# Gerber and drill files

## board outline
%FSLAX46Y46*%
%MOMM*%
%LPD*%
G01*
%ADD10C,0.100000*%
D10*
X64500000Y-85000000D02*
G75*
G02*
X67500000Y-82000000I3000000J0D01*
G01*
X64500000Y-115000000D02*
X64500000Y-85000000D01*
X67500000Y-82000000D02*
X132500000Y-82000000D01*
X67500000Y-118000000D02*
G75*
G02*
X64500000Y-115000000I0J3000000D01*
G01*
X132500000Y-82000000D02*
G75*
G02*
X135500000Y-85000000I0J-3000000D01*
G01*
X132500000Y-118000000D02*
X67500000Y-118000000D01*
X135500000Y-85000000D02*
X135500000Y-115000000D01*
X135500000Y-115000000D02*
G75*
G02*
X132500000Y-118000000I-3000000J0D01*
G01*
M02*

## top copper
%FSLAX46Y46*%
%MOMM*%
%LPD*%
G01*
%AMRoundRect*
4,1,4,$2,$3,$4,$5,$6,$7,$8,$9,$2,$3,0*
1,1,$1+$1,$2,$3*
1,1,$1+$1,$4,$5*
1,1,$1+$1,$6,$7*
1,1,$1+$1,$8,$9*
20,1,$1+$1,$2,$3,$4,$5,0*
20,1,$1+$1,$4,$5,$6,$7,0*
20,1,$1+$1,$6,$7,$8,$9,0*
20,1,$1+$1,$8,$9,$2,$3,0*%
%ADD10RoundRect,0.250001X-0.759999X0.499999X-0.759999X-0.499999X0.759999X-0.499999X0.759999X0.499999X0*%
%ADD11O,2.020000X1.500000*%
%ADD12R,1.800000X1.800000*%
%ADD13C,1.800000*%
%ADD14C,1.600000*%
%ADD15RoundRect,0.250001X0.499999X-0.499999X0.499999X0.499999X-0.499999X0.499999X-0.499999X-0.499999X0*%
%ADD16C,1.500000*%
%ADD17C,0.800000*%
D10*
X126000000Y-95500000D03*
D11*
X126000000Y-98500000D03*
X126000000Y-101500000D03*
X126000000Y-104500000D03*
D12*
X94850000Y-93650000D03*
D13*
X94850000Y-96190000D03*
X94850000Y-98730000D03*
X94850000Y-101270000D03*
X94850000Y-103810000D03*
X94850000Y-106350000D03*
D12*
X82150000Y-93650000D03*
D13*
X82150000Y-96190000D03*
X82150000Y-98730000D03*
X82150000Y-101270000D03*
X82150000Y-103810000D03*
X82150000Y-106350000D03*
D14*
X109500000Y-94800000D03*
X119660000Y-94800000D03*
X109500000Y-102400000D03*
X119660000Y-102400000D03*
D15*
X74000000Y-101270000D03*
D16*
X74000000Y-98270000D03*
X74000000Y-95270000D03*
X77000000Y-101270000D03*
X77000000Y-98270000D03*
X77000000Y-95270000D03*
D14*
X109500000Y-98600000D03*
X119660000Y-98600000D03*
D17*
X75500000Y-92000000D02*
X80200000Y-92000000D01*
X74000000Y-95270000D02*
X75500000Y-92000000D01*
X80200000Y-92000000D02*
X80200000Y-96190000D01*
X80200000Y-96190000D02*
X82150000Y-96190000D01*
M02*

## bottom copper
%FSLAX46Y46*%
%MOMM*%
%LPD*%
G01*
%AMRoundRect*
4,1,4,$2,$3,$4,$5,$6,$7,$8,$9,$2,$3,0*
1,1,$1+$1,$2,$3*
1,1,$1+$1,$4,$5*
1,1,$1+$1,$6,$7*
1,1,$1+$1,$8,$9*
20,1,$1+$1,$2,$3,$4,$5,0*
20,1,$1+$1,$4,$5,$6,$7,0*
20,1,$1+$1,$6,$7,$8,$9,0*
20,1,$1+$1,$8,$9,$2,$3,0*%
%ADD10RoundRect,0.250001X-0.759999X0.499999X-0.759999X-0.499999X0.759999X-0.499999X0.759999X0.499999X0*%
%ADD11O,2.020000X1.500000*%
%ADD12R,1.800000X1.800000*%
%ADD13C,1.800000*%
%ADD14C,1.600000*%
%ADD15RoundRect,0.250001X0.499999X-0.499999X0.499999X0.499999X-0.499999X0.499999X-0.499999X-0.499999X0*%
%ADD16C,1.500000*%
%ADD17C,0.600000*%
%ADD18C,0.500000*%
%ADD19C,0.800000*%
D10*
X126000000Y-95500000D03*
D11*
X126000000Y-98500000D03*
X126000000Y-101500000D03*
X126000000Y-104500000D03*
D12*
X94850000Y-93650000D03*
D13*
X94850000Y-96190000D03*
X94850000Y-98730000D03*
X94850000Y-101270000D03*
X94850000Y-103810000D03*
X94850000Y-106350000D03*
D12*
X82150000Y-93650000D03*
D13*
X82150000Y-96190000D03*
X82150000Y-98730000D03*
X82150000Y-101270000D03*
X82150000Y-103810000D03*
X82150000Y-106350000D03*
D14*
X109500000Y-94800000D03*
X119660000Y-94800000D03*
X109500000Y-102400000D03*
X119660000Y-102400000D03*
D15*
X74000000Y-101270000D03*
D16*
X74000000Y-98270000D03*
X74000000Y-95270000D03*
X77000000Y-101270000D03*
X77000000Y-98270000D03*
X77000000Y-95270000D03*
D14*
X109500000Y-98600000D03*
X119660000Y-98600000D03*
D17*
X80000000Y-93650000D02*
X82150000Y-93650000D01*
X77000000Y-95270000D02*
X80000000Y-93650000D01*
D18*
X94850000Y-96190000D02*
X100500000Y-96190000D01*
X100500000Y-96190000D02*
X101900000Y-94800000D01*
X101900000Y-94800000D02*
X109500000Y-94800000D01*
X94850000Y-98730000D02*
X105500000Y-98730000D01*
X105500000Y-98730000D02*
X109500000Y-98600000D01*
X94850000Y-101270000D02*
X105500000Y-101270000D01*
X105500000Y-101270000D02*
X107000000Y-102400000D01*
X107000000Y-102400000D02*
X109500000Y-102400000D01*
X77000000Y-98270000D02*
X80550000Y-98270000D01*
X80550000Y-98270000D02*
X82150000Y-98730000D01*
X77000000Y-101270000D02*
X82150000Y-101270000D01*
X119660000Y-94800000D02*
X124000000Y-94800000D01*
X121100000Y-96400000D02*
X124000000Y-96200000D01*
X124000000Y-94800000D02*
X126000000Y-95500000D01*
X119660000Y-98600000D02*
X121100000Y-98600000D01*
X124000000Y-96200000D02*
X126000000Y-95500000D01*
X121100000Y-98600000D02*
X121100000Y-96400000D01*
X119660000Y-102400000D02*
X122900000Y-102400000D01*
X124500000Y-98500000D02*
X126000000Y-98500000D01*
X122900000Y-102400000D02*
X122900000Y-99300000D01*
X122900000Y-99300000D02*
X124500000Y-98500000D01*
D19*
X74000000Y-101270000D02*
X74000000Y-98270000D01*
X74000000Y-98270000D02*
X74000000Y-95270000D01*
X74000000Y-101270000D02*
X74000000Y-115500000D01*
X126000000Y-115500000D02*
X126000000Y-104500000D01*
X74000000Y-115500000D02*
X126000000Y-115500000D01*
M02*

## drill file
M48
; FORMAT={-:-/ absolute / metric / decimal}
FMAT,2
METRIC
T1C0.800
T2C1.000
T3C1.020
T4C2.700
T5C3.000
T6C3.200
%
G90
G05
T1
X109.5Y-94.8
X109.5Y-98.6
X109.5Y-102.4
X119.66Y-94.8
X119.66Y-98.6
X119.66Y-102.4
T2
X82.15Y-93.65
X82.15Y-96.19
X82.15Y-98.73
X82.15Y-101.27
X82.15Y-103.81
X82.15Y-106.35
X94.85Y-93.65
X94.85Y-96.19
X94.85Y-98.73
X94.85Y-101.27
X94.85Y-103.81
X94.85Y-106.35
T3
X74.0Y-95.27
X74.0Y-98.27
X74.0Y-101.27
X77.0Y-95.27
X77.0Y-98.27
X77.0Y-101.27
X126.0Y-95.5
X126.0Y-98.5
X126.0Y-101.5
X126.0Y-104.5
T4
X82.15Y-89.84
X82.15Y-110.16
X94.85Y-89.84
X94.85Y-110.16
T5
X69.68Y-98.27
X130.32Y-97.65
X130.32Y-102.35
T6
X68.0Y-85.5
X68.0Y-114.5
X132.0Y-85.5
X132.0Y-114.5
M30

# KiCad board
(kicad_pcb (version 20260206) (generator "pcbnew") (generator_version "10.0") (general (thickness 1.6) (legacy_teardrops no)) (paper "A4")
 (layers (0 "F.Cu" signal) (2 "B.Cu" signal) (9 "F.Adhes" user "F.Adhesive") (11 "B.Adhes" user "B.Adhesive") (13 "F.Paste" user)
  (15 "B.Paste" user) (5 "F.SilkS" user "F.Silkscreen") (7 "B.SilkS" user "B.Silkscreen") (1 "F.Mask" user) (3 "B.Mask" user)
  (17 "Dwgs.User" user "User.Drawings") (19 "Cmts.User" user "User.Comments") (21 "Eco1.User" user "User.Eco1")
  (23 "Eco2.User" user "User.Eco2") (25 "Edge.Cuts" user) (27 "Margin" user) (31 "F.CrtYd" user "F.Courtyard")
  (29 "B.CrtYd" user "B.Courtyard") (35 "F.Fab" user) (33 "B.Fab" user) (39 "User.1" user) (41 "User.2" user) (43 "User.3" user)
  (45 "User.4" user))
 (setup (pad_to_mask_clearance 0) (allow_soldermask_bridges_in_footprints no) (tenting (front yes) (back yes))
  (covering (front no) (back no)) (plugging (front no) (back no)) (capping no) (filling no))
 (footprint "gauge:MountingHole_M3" (layer "F.Cu") (at 68 114.5)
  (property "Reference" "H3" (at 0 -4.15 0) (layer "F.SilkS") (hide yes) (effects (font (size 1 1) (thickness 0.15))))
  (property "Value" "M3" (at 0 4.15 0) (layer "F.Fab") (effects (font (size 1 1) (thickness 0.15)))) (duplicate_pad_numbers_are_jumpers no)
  (pad "" np_thru_hole circle (at 0 0) (size 3.2 3.2) (drill 3.2) (layers "*.Cu" "*.Mask")))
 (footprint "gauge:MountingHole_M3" (layer "F.Cu") (at 68 85.5)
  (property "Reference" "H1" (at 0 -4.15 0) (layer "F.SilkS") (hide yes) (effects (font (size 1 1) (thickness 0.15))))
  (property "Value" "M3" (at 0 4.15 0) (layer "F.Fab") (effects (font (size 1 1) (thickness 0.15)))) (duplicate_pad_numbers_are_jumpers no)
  (pad "" np_thru_hole circle (at 0 0) (size 3.2 3.2) (drill 3.2) (layers "*.Cu" "*.Mask")))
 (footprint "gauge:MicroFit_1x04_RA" (layer "F.Cu") (at 126 95.5 -90)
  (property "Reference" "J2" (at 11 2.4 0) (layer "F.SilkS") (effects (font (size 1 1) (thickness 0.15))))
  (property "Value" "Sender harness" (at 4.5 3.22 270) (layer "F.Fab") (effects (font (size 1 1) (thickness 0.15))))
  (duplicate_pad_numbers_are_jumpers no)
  (pad "" np_thru_hole circle (at 2.15 -4.32 270) (size 3 3) (drill 3) (layers "*.Cu" "*.Mask"))
  (pad "" np_thru_hole circle (at 6.85 -4.32 270) (size 3 3) (drill 3) (layers "*.Cu" "*.Mask"))
  (pad "1" thru_hole roundrect (at 0 0 270) (size 1.5 2.02) (drill 1.02) (layers "*.Cu" "*.Mask") (remove_unused_layers no)
   (roundrect_rratio 0.166667) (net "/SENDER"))
  (pad "2" thru_hole oval (at 3 0 270) (size 1.5 2.02) (drill 1.02) (layers "*.Cu" "*.Mask") (remove_unused_layers no) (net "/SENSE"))
  (pad "3" thru_hole oval (at 6 0 270) (size 1.5 2.02) (drill 1.02) (layers "*.Cu" "*.Mask") (remove_unused_layers no)
   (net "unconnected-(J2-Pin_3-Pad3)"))
  (pad "4" thru_hole oval (at 9 0 270) (size 1.5 2.02) (drill 1.02) (layers "*.Cu" "*.Mask") (remove_unused_layers no) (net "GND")))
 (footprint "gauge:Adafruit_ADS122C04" (layer "F.Cu") (at 88.5 100 -90)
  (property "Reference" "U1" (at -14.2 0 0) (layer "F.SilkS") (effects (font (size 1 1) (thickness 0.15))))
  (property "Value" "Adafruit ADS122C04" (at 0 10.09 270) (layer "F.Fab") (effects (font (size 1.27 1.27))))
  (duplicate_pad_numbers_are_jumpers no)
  (pad "" np_thru_hole circle (at -10.16 -6.35 270) (size 2.7 2.7) (drill 2.7) (layers "*.Cu"))
  (pad "" np_thru_hole circle (at -10.16 6.35 270) (size 2.7 2.7) (drill 2.7) (layers "*.Cu"))
  (pad "" np_thru_hole circle (at 10.16 -6.35 270) (size 2.7 2.7) (drill 2.7) (layers "*.Cu"))
  (pad "" np_thru_hole circle (at 10.16 6.35 270) (size 2.7 2.7) (drill 2.7) (layers "*.Cu"))
  (pad "1" thru_hole rect (at -6.35 -6.35 270) (size 1.8 1.8) (drill 1) (layers "*.Cu" "*.Mask") (remove_unused_layers no)
   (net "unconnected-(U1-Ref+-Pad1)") (thermal_bridge_angle 45))
  (pad "2" thru_hole circle (at -3.81 -6.35 270) (size 1.8 1.8) (drill 1) (layers "*.Cu" "*.Mask") (remove_unused_layers no) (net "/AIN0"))
  (pad "3" thru_hole circle (at -1.27 -6.35 270) (size 1.8 1.8) (drill 1) (layers "*.Cu" "*.Mask") (remove_unused_layers no) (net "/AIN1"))
  (pad "4" thru_hole circle (at 1.27 -6.35 270) (size 1.8 1.8) (drill 1) (layers "*.Cu" "*.Mask") (remove_unused_layers no) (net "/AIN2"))
  (pad "5" thru_hole circle (at 3.81 -6.35 270) (size 1.8 1.8) (drill 1) (layers "*.Cu" "*.Mask") (remove_unused_layers no)
   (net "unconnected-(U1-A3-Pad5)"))
  (pad "6" thru_hole circle (at 6.35 -6.35 270) (size 1.8 1.8) (drill 1) (layers "*.Cu" "*.Mask") (remove_unused_layers no)
   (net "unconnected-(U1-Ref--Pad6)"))
  (pad "7" thru_hole rect (at -6.35 6.35 270) (size 1.8 1.8) (drill 1) (layers "*.Cu" "*.Mask") (remove_unused_layers no) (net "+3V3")
   (thermal_bridge_angle 45))
  (pad "8" thru_hole circle (at -3.81 6.35 270) (size 1.8 1.8) (drill 1) (layers "*.Cu" "*.Mask") (remove_unused_layers no) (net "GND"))
  (pad "9" thru_hole circle (at -1.27 6.35 270) (size 1.8 1.8) (drill 1) (layers "*.Cu" "*.Mask") (remove_unused_layers no) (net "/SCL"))
  (pad "10" thru_hole circle (at 1.27 6.35 270) (size 1.8 1.8) (drill 1) (layers "*.Cu" "*.Mask") (remove_unused_layers no) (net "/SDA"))
  (pad "11" thru_hole circle (at 3.81 6.35 270) (size 1.8 1.8) (drill 1) (layers "*.Cu" "*.Mask") (remove_unused_layers no)
   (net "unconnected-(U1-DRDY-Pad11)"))
  (pad "12" thru_hole circle (at 6.35 6.35 270) (size 1.8 1.8) (drill 1) (layers "*.Cu" "*.Mask") (remove_unused_layers no)
   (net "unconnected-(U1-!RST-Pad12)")))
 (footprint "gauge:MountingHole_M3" (layer "F.Cu") (at 132 114.5)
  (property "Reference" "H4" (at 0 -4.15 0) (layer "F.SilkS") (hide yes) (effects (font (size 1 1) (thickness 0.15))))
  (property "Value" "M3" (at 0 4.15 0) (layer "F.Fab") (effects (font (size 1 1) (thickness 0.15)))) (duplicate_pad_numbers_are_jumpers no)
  (pad "" np_thru_hole circle (at 0 0) (size 3.2 3.2) (drill 3.2) (layers "*.Cu" "*.Mask")))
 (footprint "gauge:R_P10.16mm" (layer "F.Cu") (at 109.5 94.8)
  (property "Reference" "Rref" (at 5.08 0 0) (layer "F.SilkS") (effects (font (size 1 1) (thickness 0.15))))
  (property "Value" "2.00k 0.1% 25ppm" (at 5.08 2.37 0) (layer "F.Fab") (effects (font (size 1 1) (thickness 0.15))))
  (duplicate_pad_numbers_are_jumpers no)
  (pad "1" thru_hole circle (at 0 0) (size 1.6 1.6) (drill 0.8) (layers "*.Cu" "*.Mask") (remove_unused_layers no) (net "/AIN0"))
  (pad "2" thru_hole circle (at 10.16 0) (size 1.6 1.6) (drill 0.8) (layers "*.Cu" "*.Mask") (remove_unused_layers no) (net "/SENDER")))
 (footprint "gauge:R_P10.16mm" (layer "F.Cu") (at 109.5 102.4)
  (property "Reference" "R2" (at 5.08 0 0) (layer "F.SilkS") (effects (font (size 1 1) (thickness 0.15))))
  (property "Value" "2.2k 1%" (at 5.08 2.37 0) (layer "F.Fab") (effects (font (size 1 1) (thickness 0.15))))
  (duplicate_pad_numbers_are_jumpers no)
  (pad "1" thru_hole circle (at 0 0) (size 1.6 1.6) (drill 0.8) (layers "*.Cu" "*.Mask") (remove_unused_layers no) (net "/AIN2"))
  (pad "2" thru_hole circle (at 10.16 0) (size 1.6 1.6) (drill 0.8) (layers "*.Cu" "*.Mask") (remove_unused_layers no) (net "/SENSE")))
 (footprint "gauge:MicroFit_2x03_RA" (layer "F.Cu") (at 74 101.27 90)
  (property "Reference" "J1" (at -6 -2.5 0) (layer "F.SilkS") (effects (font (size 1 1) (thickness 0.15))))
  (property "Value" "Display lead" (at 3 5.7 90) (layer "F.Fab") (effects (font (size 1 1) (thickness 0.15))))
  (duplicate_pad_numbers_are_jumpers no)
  (pad "" np_thru_hole circle (at 3 -4.32 90) (size 3 3) (drill 3) (layers "*.Cu" "*.Mask"))
  (pad "1" thru_hole roundrect (at 0 0 90) (size 1.5 1.5) (drill 1.02) (layers "*.Cu" "*.Mask") (remove_unused_layers no)
   (roundrect_rratio 0.166667) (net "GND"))
  (pad "2" thru_hole circle (at 3 0 90) (size 1.5 1.5) (drill 1.02) (layers "*.Cu" "*.Mask") (remove_unused_layers no) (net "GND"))
  (pad "3" thru_hole circle (at 6 0 90) (size 1.5 1.5) (drill 1.02) (layers "*.Cu" "*.Mask") (remove_unused_layers no) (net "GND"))
  (pad "4" thru_hole circle (at 0 3 90) (size 1.5 1.5) (drill 1.02) (layers "*.Cu" "*.Mask") (remove_unused_layers no) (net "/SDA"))
  (pad "5" thru_hole circle (at 3 3 90) (size 1.5 1.5) (drill 1.02) (layers "*.Cu" "*.Mask") (remove_unused_layers no) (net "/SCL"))
  (pad "6" thru_hole circle (at 6 3 90) (size 1.5 1.5) (drill 1.02) (layers "*.Cu" "*.Mask") (remove_unused_layers no) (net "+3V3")))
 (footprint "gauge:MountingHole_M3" (layer "F.Cu") (at 132 85.5)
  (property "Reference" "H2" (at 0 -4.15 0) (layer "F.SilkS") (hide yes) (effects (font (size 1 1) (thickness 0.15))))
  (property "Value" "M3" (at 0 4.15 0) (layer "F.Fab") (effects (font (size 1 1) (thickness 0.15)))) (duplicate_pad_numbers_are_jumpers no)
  (pad "" np_thru_hole circle (at 0 0) (size 3.2 3.2) (drill 3.2) (layers "*.Cu" "*.Mask")))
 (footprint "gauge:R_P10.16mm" (layer "F.Cu") (at 109.5 98.6)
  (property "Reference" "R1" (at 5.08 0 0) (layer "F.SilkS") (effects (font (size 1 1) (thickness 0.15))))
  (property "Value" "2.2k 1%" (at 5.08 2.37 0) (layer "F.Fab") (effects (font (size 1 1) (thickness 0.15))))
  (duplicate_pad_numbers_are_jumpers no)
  (pad "1" thru_hole circle (at 0 0) (size 1.6 1.6) (drill 0.8) (layers "*.Cu" "*.Mask") (remove_unused_layers no) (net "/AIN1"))
  (pad "2" thru_hole circle (at 10.16 0) (size 1.6 1.6) (drill 0.8) (layers "*.Cu" "*.Mask") (remove_unused_layers no) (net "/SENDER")))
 (gr_arc (start 64.5 85) (mid 65.37868 82.87868) (end 67.5 82) (stroke (width 0.1) (type default)) (layer "Edge.Cuts"))
 (gr_line (start 64.5 115) (end 64.5 85) (stroke (width 0.1) (type default)) (layer "Edge.Cuts"))
 (gr_line (start 67.5 82) (end 132.5 82) (stroke (width 0.1) (type default)) (layer "Edge.Cuts"))
 (gr_arc (start 67.5 118) (mid 65.37868 117.12132) (end 64.5 115) (stroke (width 0.1) (type default)) (layer "Edge.Cuts"))
 (gr_arc (start 132.5 82) (mid 134.62132 82.87868) (end 135.5 85) (stroke (width 0.1) (type default)) (layer "Edge.Cuts"))
 (gr_line (start 132.5 118) (end 67.5 118) (stroke (width 0.1) (type default)) (layer "Edge.Cuts"))
 (gr_line (start 135.5 85) (end 135.5 115) (stroke (width 0.1) (type default)) (layer "Edge.Cuts"))
 (gr_arc (start 135.5 115) (mid 134.62132 117.12132) (end 132.5 118) (stroke (width 0.1) (type default)) (layer "Edge.Cuts"))
 (segment (start 80 93.65) (end 82.15 93.65) (width 0.6) (layer "B.Cu") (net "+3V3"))
 (segment (start 77 95.27) (end 80 93.65) (width 0.6) (layer "B.Cu") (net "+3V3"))
 (segment (start 94.85 96.19) (end 100.5 96.19) (width 0.5) (layer "B.Cu") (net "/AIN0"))
 (segment (start 100.5 96.19) (end 101.9 94.8) (width 0.5) (layer "B.Cu") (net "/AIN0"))
 (segment (start 101.9 94.8) (end 109.5 94.8) (width 0.5) (layer "B.Cu") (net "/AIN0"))
 (segment (start 94.85 98.73) (end 105.5 98.73) (width 0.5) (layer "B.Cu") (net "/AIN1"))
 (segment (start 105.5 98.73) (end 109.5 98.6) (width 0.5) (layer "B.Cu") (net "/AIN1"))
 (segment (start 94.85 101.27) (end 105.5 101.27) (width 0.5) (layer "B.Cu") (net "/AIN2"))
 (segment (start 105.5 101.27) (end 107 102.4) (width 0.5) (layer "B.Cu") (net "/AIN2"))
 (segment (start 107 102.4) (end 109.5 102.4) (width 0.5) (layer "B.Cu") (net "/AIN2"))
 (segment (start 77 98.27) (end 80.55 98.27) (width 0.5) (layer "B.Cu") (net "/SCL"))
 (segment (start 80.55 98.27) (end 82.15 98.73) (width 0.5) (layer "B.Cu") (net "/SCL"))
 (segment (start 77 101.27) (end 82.15 101.27) (width 0.5) (layer "B.Cu") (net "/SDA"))
 (segment (start 119.66 94.8) (end 124 94.8) (width 0.5) (layer "B.Cu") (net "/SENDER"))
 (segment (start 121.1 96.4) (end 124 96.2) (width 0.5) (layer "B.Cu") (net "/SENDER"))
 (segment (start 124 94.8) (end 126 95.5) (width 0.5) (layer "B.Cu") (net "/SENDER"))
 (segment (start 119.66 98.6) (end 121.1 98.6) (width 0.5) (layer "B.Cu") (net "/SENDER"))
 (segment (start 124 96.2) (end 126 95.5) (width 0.5) (layer "B.Cu") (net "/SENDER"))
 (segment (start 121.1 98.6) (end 121.1 96.4) (width 0.5) (layer "B.Cu") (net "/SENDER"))
 (segment (start 119.66 102.4) (end 122.9 102.4) (width 0.5) (layer "B.Cu") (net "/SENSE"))
 (segment (start 124.5 98.5) (end 126 98.5) (width 0.5) (layer "B.Cu") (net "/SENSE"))
 (segment (start 122.9 102.4) (end 122.9 99.3) (width 0.5) (layer "B.Cu") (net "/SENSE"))
 (segment (start 122.9 99.3) (end 124.5 98.5) (width 0.5) (layer "B.Cu") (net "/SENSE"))
 (segment (start 75.5 92) (end 80.2 92) (width 0.8) (layer "F.Cu") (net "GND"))
 (segment (start 74 95.27) (end 75.5 92) (width 0.8) (layer "F.Cu") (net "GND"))
 (segment (start 80.2 92) (end 80.2 96.19) (width 0.8) (layer "F.Cu") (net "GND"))
 (segment (start 80.2 96.19) (end 82.15 96.19) (width 0.8) (layer "F.Cu") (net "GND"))
 (segment (start 74 101.27) (end 74 98.27) (width 0.8) (layer "B.Cu") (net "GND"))
 (segment (start 74 98.27) (end 74 95.27) (width 0.8) (layer "B.Cu") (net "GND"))
 (segment (start 74 101.27) (end 74 115.5) (width 0.8) (layer "B.Cu") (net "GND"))
 (segment (start 126 115.5) (end 126 104.5) (width 0.8) (layer "B.Cu") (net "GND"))
 (segment (start 74 115.5) (end 126 115.5) (width 0.8) (layer "B.Cu") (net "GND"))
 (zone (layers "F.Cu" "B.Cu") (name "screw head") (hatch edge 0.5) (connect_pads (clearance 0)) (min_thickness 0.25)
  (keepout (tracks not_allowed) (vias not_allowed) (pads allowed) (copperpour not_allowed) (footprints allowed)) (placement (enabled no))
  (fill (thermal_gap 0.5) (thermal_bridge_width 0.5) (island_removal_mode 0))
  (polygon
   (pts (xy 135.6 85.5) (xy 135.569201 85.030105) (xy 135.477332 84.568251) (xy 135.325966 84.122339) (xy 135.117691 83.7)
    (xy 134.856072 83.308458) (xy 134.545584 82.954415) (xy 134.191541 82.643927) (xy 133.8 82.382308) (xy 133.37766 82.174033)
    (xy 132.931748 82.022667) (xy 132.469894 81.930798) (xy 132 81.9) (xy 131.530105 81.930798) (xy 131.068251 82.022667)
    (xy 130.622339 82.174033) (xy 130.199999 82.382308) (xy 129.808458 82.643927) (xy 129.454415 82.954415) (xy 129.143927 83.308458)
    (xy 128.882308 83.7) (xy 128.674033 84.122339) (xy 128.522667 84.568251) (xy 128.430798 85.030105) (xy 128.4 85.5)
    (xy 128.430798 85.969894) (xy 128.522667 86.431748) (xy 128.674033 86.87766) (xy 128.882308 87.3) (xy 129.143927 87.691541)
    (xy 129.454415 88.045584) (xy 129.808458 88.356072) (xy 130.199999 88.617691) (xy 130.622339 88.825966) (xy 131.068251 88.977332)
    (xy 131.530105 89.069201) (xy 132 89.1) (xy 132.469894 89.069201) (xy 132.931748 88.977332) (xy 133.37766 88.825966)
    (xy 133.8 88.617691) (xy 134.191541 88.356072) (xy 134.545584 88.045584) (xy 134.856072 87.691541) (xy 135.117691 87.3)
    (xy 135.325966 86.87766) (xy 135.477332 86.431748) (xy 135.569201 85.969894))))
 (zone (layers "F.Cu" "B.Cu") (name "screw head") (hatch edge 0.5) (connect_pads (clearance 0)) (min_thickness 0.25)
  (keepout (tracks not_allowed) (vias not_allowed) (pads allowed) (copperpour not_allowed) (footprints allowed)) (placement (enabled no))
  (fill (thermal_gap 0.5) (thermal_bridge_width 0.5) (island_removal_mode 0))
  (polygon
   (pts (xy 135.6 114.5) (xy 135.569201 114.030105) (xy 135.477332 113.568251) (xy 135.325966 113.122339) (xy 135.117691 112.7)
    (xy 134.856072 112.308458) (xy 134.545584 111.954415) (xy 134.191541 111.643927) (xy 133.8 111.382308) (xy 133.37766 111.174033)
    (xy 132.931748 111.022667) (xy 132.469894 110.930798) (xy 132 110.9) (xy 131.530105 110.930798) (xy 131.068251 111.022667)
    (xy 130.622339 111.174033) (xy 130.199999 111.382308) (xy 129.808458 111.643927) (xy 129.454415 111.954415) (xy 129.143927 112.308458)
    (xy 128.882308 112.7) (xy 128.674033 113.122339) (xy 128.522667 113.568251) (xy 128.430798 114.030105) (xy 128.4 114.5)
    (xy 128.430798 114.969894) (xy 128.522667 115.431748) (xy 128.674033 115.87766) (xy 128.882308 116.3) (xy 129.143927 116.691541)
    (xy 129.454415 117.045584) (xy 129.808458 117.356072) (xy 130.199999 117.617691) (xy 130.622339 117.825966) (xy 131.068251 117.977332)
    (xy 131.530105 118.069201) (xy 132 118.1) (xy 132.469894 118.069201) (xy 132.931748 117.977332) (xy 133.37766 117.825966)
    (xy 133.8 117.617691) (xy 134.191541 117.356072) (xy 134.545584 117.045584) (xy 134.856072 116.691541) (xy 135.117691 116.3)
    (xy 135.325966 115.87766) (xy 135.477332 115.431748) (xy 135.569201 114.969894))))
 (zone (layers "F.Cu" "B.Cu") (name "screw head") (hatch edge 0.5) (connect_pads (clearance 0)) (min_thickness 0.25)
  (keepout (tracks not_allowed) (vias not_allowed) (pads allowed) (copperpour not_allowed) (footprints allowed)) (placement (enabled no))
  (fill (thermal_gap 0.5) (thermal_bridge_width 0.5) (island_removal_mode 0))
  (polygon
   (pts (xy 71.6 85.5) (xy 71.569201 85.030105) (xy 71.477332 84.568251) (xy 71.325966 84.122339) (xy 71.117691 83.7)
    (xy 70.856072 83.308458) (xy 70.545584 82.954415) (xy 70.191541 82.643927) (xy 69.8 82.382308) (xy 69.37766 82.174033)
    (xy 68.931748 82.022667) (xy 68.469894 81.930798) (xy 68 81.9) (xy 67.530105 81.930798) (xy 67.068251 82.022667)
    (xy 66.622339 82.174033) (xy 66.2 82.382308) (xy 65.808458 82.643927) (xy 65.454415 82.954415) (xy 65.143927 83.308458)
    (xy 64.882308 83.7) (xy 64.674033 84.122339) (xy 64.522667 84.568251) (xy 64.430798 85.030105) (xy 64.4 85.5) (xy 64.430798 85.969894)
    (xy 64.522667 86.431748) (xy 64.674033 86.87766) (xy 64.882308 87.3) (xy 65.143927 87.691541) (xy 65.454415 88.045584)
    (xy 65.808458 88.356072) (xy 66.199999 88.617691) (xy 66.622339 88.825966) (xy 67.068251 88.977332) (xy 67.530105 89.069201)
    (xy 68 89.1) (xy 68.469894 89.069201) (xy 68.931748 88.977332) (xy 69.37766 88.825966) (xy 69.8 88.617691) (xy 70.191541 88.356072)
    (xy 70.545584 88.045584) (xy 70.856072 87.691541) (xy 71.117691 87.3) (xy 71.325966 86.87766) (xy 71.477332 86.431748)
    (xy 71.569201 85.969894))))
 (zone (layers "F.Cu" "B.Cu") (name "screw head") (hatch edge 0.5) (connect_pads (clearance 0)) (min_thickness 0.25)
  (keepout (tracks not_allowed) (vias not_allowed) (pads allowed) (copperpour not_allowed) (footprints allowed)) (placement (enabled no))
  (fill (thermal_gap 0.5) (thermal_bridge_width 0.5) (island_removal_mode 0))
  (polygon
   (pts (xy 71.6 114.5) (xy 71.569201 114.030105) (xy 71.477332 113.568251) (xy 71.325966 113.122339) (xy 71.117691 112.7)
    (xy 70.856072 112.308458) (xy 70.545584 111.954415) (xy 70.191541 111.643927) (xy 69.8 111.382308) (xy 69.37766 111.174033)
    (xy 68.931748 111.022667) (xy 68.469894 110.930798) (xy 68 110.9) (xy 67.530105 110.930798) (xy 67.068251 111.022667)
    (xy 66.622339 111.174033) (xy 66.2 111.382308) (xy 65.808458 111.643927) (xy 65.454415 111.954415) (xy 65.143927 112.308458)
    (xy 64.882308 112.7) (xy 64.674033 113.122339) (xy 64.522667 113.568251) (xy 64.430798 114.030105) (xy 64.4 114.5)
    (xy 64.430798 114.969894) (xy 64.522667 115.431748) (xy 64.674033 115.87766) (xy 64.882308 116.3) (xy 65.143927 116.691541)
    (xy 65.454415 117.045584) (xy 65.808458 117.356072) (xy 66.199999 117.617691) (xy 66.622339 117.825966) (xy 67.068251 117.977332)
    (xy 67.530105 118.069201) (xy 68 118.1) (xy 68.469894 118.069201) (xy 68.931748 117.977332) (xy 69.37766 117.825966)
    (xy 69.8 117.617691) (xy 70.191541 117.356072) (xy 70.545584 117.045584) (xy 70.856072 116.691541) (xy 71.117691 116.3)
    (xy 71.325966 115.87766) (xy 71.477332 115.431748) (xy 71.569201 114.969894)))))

